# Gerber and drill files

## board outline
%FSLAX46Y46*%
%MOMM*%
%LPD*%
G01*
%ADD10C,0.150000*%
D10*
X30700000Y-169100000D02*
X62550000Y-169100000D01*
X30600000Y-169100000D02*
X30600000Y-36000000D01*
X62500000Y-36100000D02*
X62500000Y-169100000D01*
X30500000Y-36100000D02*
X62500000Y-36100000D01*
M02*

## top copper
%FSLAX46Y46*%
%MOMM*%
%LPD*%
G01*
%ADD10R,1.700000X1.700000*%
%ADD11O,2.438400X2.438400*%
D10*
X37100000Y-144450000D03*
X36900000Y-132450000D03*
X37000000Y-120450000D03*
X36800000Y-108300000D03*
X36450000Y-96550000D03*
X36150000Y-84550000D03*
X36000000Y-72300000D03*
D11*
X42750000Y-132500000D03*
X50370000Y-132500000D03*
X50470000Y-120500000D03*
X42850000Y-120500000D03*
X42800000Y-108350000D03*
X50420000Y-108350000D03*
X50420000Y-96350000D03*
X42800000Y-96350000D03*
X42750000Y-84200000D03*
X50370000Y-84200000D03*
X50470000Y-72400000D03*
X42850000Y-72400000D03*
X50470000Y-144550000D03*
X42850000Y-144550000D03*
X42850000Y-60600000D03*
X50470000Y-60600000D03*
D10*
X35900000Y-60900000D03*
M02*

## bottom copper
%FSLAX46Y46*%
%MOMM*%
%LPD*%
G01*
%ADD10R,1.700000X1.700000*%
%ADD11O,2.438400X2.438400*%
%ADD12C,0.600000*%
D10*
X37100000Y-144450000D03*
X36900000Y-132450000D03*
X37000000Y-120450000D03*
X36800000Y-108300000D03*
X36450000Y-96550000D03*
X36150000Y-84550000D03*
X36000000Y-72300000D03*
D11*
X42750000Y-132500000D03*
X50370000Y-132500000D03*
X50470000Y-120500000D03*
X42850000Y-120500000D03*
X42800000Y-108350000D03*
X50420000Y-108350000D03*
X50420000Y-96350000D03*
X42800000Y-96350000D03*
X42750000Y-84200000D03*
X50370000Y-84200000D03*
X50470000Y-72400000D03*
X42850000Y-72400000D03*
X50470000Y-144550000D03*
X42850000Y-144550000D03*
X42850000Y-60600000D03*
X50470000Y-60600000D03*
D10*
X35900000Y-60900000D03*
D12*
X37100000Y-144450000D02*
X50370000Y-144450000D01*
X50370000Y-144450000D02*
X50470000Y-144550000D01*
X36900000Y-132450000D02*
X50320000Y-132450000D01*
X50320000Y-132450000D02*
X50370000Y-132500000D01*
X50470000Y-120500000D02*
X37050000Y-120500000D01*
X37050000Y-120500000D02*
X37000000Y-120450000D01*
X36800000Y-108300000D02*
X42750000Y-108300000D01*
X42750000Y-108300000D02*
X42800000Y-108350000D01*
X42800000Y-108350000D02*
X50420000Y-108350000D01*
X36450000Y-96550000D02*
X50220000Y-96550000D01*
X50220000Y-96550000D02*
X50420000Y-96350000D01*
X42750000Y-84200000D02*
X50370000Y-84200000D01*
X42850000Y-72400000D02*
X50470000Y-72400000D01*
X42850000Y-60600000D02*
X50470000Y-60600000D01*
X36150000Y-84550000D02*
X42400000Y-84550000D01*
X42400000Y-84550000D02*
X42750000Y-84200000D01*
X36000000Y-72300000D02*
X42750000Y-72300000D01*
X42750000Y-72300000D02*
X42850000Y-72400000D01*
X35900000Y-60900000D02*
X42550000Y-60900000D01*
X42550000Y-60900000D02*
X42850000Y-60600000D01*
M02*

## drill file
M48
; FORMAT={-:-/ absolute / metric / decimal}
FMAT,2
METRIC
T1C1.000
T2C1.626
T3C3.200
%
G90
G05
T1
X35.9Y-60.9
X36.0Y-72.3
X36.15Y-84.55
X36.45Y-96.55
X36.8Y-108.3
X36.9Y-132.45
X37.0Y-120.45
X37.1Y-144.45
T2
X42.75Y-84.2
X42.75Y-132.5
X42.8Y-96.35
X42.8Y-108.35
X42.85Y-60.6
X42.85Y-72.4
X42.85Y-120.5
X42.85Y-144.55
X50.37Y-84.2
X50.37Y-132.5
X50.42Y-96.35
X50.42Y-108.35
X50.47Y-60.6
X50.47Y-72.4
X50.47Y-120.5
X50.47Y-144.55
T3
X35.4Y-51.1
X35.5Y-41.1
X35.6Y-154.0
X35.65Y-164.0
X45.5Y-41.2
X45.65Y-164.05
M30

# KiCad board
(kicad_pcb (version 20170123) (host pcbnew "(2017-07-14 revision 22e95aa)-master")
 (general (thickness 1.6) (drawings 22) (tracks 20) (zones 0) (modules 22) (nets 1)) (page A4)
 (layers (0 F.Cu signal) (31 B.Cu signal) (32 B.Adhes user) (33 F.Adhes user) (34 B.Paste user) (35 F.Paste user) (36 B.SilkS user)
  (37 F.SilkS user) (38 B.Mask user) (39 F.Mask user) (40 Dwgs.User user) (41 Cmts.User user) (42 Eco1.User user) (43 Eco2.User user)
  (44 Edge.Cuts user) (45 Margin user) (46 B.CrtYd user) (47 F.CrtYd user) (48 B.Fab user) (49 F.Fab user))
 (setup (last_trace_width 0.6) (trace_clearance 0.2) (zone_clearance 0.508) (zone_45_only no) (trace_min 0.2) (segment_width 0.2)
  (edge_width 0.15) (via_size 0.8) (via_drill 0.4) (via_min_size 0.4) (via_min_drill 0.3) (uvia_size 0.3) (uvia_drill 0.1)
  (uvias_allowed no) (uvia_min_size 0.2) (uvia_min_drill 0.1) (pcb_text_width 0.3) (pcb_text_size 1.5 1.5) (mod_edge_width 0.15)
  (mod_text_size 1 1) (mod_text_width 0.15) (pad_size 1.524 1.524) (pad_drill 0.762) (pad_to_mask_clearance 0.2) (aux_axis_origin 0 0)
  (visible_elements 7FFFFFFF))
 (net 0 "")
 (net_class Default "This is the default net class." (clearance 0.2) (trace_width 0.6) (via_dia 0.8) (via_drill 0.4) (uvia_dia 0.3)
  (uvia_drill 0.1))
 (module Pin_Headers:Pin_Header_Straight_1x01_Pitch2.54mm (layer F.Cu) (at 37.1 144.45)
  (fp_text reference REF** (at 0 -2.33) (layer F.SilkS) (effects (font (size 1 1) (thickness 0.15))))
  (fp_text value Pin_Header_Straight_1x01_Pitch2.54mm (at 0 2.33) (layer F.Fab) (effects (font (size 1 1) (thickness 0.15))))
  (pad 1 thru_hole rect (at 0 0) (size 1.7 1.7) (drill 1) (layers *.Cu *.Mask)))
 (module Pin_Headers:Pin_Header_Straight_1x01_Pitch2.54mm (layer F.Cu) (at 36.9 132.45)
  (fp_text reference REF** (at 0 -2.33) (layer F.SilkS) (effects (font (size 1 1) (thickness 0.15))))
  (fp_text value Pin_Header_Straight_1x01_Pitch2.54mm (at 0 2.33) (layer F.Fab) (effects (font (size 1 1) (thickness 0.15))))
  (pad 1 thru_hole rect (at 0 0) (size 1.7 1.7) (drill 1) (layers *.Cu *.Mask)))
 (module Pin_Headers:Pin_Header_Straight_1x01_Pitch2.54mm (layer F.Cu) (at 37 120.45)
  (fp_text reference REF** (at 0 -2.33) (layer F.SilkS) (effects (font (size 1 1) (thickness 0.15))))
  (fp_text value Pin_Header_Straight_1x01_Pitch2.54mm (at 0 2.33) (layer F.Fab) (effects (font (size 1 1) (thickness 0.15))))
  (pad 1 thru_hole rect (at 0 0) (size 1.7 1.7) (drill 1) (layers *.Cu *.Mask)))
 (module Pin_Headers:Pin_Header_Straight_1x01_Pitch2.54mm (layer F.Cu) (at 36.8 108.3)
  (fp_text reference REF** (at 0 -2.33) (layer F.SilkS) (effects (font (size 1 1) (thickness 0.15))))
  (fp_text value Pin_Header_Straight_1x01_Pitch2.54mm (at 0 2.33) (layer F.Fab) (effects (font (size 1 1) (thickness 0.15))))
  (pad 1 thru_hole rect (at 0 0) (size 1.7 1.7) (drill 1) (layers *.Cu *.Mask)))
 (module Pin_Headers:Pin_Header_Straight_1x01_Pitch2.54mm (layer F.Cu) (at 36.45 96.55)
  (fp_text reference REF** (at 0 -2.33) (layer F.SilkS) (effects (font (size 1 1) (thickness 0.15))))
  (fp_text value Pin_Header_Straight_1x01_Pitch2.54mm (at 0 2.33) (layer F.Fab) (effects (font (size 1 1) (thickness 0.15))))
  (pad 1 thru_hole rect (at 0 0) (size 1.7 1.7) (drill 1) (layers *.Cu *.Mask)))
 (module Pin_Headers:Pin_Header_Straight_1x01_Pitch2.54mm (layer F.Cu) (at 36.15 84.55)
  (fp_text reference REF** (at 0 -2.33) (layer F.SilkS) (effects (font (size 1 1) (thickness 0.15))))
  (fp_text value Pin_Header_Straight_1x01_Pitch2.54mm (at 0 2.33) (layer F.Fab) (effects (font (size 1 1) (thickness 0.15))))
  (pad 1 thru_hole rect (at 0 0) (size 1.7 1.7) (drill 1) (layers *.Cu *.Mask)))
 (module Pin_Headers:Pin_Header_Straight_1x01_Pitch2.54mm (layer F.Cu) (at 36 72.3)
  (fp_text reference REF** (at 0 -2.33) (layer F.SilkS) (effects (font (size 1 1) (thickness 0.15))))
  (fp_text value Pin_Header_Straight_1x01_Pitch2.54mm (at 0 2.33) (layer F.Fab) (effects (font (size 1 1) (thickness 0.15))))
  (pad 1 thru_hole rect (at 0 0) (size 1.7 1.7) (drill 1) (layers *.Cu *.Mask)))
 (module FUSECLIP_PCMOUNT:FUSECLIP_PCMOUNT (layer F.Cu) (at 42.75 132.5)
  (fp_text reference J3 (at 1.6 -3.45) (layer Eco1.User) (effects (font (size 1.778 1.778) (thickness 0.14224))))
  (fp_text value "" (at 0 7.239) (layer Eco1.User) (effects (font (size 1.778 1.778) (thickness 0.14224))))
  (pad 1 thru_hole oval (at 0 0) (size 2.4384 2.4384) (drill 1.6256) (layers *.Cu *.Mask))
  (pad 2 thru_hole oval (at 7.62 0) (size 2.4384 2.4384) (drill 1.6256) (layers *.Cu *.Mask)))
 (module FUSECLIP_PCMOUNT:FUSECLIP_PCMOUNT (layer F.Cu) (at 42.85 120.5)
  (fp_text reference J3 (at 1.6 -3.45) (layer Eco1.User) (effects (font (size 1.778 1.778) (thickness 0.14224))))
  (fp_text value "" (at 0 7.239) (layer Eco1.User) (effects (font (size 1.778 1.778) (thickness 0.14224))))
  (pad 2 thru_hole oval (at 7.62 0) (size 2.4384 2.4384) (drill 1.6256) (layers *.Cu *.Mask))
  (pad 1 thru_hole oval (at 0 0) (size 2.4384 2.4384) (drill 1.6256) (layers *.Cu *.Mask)))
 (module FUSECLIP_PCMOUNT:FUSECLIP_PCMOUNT (layer F.Cu) (at 42.8 108.35)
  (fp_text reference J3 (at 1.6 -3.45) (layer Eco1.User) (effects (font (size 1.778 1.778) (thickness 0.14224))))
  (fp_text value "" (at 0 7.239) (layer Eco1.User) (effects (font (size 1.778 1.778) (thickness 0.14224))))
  (pad 1 thru_hole oval (at 0 0) (size 2.4384 2.4384) (drill 1.6256) (layers *.Cu *.Mask))
  (pad 2 thru_hole oval (at 7.62 0) (size 2.4384 2.4384) (drill 1.6256) (layers *.Cu *.Mask)))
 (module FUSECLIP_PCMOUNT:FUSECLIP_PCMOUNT (layer F.Cu) (at 42.8 96.35)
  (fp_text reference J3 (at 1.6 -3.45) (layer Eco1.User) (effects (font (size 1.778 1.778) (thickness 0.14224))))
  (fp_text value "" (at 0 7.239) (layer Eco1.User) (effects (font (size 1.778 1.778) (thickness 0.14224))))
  (pad 2 thru_hole oval (at 7.62 0) (size 2.4384 2.4384) (drill 1.6256) (layers *.Cu *.Mask))
  (pad 1 thru_hole oval (at 0 0) (size 2.4384 2.4384) (drill 1.6256) (layers *.Cu *.Mask)))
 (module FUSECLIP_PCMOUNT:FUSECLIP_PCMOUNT (layer F.Cu) (at 42.75 84.2)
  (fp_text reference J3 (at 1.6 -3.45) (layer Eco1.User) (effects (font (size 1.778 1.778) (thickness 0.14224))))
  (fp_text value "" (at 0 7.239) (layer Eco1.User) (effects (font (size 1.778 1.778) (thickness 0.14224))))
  (pad 1 thru_hole oval (at 0 0) (size 2.4384 2.4384) (drill 1.6256) (layers *.Cu *.Mask))
  (pad 2 thru_hole oval (at 7.62 0) (size 2.4384 2.4384) (drill 1.6256) (layers *.Cu *.Mask)))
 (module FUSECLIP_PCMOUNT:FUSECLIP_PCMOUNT (layer F.Cu) (at 42.85 72.4)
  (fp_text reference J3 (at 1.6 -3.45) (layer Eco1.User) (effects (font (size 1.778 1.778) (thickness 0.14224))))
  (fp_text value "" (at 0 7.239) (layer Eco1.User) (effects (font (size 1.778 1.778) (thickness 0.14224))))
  (pad 2 thru_hole oval (at 7.62 0) (size 2.4384 2.4384) (drill 1.6256) (layers *.Cu *.Mask))
  (pad 1 thru_hole oval (at 0 0) (size 2.4384 2.4384) (drill 1.6256) (layers *.Cu *.Mask)))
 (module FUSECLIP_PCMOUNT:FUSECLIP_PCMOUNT (layer F.Cu) (at 42.85 144.55)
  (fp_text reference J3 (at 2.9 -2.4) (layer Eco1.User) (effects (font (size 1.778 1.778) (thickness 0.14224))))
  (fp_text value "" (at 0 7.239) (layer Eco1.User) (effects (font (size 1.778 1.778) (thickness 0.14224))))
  (pad 2 thru_hole oval (at 7.62 0) (size 2.4384 2.4384) (drill 1.6256) (layers *.Cu *.Mask))
  (pad 1 thru_hole oval (at 0 0) (size 2.4384 2.4384) (drill 1.6256) (layers *.Cu *.Mask)))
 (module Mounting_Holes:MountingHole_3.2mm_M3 (layer F.Cu) (at 35.6 154)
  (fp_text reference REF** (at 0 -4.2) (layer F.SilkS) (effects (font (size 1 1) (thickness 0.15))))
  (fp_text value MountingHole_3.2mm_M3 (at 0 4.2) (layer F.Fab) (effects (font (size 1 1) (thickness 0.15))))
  (pad 1 np_thru_hole circle (at 0 0) (size 3.2 3.2) (drill 3.2) (layers *.Cu *.Mask)))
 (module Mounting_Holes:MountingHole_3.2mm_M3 (layer F.Cu) (at 35.4 51.1)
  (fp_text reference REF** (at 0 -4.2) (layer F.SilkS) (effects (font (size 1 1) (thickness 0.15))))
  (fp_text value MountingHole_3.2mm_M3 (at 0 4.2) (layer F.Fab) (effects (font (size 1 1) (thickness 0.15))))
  (pad 1 np_thru_hole circle (at 0 0) (size 3.2 3.2) (drill 3.2) (layers *.Cu *.Mask)))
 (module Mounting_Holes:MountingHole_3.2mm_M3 (layer F.Cu) (at 45.65 164.05)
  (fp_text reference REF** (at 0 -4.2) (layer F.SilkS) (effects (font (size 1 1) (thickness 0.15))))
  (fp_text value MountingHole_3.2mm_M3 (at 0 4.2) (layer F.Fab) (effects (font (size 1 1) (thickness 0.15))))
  (pad 1 np_thru_hole circle (at 0 0) (size 3.2 3.2) (drill 3.2) (layers *.Cu *.Mask)))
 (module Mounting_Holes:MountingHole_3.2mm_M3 (layer F.Cu) (at 35.5 41.1)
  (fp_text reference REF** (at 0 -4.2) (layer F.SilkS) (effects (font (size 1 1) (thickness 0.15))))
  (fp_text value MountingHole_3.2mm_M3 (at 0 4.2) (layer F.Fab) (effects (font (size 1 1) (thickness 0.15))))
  (pad 1 np_thru_hole circle (at 0 0) (size 3.2 3.2) (drill 3.2) (layers *.Cu *.Mask)))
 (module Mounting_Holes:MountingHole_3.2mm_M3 (layer F.Cu) (at 35.65 164)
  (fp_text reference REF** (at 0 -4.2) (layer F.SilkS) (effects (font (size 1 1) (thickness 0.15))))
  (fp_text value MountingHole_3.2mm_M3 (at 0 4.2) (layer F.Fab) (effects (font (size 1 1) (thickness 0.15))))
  (pad 1 np_thru_hole circle (at 0 0) (size 3.2 3.2) (drill 3.2) (layers *.Cu *.Mask)))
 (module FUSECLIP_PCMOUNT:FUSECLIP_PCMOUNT (layer F.Cu) (at 42.85 60.6)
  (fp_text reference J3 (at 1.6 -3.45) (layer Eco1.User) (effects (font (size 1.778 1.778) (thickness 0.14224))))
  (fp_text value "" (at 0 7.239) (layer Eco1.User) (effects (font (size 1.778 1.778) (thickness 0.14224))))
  (pad 1 thru_hole oval (at 0 0) (size 2.4384 2.4384) (drill 1.6256) (layers *.Cu *.Mask))
  (pad 2 thru_hole oval (at 7.62 0) (size 2.4384 2.4384) (drill 1.6256) (layers *.Cu *.Mask)))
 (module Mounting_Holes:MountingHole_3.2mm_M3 (layer F.Cu) (at 45.5 41.2)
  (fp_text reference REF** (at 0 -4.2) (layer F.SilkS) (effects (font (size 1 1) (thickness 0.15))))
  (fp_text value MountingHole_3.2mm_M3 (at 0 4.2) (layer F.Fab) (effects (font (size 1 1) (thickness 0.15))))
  (pad 1 np_thru_hole circle (at 0 0) (size 3.2 3.2) (drill 3.2) (layers *.Cu *.Mask)))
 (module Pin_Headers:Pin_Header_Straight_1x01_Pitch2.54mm (layer F.Cu) (at 35.9 60.9)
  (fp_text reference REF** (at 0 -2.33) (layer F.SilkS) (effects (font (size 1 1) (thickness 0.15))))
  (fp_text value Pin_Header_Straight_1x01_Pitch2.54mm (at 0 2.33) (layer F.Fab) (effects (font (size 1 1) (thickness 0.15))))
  (pad 1 thru_hole rect (at 0 0) (size 1.7 1.7) (drill 1) (layers *.Cu *.Mask)))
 (gr_line (start 30.7 169.1) (end 62.55 169.1) (angle 90) (layer Edge.Cuts) (width 0.15))
 (gr_line (start 30.6 169.1) (end 30.6 36) (angle 90) (layer Edge.Cuts) (width 0.15))
 (gr_line (start 62.5 36.1) (end 62.5 169.1) (angle 90) (layer Edge.Cuts) (width 0.15))
 (gr_line (start 30.5 36.1) (end 62.5 36.1) (angle 90) (layer Edge.Cuts) (width 0.15))
 (segment (start 37.1 144.45) (end 50.37 144.45) (width 0.6) (layer B.Cu) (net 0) (status C00000))
 (segment (start 50.37 144.45) (end 50.47 144.55) (width 0.6) (layer B.Cu) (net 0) (status C00000))
 (segment (start 36.9 132.45) (end 50.32 132.45) (width 0.6) (layer B.Cu) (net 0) (status C00000))
 (segment (start 50.32 132.45) (end 50.37 132.5) (width 0.6) (layer B.Cu) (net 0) (status C00000))
 (segment (start 50.47 120.5) (end 37.05 120.5) (width 0.6) (layer B.Cu) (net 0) (status C00000))
 (segment (start 37.05 120.5) (end 37 120.45) (width 0.6) (layer B.Cu) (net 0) (status C00000))
 (segment (start 36.8 108.3) (end 42.75 108.3) (width 0.6) (layer B.Cu) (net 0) (status C00000))
 (segment (start 42.75 108.3) (end 42.8 108.35) (width 0.6) (layer B.Cu) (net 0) (status C00000))
 (segment (start 42.8 108.35) (end 50.42 108.35) (width 0.6) (layer B.Cu) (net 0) (status C00000))
 (segment (start 36.45 96.55) (end 50.22 96.55) (width 0.6) (layer B.Cu) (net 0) (status C00000))
 (segment (start 50.22 96.55) (end 50.42 96.35) (width 0.6) (layer B.Cu) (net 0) (status C00000))
 (segment (start 42.75 84.2) (end 50.37 84.2) (width 0.6) (layer B.Cu) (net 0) (status C00000))
 (segment (start 42.85 72.4) (end 50.47 72.4) (width 0.6) (layer B.Cu) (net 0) (status C00000))
 (segment (start 42.85 60.6) (end 50.47 60.6) (width 0.6) (layer B.Cu) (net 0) (status C00000))
 (segment (start 36.15 84.55) (end 42.4 84.55) (width 0.6) (layer B.Cu) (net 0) (status C00000))
 (segment (start 42.4 84.55) (end 42.75 84.2) (width 0.6) (layer B.Cu) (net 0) (status C00000))
 (segment (start 36 72.3) (end 42.75 72.3) (width 0.6) (layer B.Cu) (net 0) (status C00000))
 (segment (start 42.75 72.3) (end 42.85 72.4) (width 0.6) (layer B.Cu) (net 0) (status C00000))
 (segment (start 35.9 60.9) (end 42.55 60.9) (width 0.6) (layer B.Cu) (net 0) (status C00000))
 (segment (start 42.55 60.9) (end 42.85 60.6) (width 0.6) (layer B.Cu) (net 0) (status C00000)))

